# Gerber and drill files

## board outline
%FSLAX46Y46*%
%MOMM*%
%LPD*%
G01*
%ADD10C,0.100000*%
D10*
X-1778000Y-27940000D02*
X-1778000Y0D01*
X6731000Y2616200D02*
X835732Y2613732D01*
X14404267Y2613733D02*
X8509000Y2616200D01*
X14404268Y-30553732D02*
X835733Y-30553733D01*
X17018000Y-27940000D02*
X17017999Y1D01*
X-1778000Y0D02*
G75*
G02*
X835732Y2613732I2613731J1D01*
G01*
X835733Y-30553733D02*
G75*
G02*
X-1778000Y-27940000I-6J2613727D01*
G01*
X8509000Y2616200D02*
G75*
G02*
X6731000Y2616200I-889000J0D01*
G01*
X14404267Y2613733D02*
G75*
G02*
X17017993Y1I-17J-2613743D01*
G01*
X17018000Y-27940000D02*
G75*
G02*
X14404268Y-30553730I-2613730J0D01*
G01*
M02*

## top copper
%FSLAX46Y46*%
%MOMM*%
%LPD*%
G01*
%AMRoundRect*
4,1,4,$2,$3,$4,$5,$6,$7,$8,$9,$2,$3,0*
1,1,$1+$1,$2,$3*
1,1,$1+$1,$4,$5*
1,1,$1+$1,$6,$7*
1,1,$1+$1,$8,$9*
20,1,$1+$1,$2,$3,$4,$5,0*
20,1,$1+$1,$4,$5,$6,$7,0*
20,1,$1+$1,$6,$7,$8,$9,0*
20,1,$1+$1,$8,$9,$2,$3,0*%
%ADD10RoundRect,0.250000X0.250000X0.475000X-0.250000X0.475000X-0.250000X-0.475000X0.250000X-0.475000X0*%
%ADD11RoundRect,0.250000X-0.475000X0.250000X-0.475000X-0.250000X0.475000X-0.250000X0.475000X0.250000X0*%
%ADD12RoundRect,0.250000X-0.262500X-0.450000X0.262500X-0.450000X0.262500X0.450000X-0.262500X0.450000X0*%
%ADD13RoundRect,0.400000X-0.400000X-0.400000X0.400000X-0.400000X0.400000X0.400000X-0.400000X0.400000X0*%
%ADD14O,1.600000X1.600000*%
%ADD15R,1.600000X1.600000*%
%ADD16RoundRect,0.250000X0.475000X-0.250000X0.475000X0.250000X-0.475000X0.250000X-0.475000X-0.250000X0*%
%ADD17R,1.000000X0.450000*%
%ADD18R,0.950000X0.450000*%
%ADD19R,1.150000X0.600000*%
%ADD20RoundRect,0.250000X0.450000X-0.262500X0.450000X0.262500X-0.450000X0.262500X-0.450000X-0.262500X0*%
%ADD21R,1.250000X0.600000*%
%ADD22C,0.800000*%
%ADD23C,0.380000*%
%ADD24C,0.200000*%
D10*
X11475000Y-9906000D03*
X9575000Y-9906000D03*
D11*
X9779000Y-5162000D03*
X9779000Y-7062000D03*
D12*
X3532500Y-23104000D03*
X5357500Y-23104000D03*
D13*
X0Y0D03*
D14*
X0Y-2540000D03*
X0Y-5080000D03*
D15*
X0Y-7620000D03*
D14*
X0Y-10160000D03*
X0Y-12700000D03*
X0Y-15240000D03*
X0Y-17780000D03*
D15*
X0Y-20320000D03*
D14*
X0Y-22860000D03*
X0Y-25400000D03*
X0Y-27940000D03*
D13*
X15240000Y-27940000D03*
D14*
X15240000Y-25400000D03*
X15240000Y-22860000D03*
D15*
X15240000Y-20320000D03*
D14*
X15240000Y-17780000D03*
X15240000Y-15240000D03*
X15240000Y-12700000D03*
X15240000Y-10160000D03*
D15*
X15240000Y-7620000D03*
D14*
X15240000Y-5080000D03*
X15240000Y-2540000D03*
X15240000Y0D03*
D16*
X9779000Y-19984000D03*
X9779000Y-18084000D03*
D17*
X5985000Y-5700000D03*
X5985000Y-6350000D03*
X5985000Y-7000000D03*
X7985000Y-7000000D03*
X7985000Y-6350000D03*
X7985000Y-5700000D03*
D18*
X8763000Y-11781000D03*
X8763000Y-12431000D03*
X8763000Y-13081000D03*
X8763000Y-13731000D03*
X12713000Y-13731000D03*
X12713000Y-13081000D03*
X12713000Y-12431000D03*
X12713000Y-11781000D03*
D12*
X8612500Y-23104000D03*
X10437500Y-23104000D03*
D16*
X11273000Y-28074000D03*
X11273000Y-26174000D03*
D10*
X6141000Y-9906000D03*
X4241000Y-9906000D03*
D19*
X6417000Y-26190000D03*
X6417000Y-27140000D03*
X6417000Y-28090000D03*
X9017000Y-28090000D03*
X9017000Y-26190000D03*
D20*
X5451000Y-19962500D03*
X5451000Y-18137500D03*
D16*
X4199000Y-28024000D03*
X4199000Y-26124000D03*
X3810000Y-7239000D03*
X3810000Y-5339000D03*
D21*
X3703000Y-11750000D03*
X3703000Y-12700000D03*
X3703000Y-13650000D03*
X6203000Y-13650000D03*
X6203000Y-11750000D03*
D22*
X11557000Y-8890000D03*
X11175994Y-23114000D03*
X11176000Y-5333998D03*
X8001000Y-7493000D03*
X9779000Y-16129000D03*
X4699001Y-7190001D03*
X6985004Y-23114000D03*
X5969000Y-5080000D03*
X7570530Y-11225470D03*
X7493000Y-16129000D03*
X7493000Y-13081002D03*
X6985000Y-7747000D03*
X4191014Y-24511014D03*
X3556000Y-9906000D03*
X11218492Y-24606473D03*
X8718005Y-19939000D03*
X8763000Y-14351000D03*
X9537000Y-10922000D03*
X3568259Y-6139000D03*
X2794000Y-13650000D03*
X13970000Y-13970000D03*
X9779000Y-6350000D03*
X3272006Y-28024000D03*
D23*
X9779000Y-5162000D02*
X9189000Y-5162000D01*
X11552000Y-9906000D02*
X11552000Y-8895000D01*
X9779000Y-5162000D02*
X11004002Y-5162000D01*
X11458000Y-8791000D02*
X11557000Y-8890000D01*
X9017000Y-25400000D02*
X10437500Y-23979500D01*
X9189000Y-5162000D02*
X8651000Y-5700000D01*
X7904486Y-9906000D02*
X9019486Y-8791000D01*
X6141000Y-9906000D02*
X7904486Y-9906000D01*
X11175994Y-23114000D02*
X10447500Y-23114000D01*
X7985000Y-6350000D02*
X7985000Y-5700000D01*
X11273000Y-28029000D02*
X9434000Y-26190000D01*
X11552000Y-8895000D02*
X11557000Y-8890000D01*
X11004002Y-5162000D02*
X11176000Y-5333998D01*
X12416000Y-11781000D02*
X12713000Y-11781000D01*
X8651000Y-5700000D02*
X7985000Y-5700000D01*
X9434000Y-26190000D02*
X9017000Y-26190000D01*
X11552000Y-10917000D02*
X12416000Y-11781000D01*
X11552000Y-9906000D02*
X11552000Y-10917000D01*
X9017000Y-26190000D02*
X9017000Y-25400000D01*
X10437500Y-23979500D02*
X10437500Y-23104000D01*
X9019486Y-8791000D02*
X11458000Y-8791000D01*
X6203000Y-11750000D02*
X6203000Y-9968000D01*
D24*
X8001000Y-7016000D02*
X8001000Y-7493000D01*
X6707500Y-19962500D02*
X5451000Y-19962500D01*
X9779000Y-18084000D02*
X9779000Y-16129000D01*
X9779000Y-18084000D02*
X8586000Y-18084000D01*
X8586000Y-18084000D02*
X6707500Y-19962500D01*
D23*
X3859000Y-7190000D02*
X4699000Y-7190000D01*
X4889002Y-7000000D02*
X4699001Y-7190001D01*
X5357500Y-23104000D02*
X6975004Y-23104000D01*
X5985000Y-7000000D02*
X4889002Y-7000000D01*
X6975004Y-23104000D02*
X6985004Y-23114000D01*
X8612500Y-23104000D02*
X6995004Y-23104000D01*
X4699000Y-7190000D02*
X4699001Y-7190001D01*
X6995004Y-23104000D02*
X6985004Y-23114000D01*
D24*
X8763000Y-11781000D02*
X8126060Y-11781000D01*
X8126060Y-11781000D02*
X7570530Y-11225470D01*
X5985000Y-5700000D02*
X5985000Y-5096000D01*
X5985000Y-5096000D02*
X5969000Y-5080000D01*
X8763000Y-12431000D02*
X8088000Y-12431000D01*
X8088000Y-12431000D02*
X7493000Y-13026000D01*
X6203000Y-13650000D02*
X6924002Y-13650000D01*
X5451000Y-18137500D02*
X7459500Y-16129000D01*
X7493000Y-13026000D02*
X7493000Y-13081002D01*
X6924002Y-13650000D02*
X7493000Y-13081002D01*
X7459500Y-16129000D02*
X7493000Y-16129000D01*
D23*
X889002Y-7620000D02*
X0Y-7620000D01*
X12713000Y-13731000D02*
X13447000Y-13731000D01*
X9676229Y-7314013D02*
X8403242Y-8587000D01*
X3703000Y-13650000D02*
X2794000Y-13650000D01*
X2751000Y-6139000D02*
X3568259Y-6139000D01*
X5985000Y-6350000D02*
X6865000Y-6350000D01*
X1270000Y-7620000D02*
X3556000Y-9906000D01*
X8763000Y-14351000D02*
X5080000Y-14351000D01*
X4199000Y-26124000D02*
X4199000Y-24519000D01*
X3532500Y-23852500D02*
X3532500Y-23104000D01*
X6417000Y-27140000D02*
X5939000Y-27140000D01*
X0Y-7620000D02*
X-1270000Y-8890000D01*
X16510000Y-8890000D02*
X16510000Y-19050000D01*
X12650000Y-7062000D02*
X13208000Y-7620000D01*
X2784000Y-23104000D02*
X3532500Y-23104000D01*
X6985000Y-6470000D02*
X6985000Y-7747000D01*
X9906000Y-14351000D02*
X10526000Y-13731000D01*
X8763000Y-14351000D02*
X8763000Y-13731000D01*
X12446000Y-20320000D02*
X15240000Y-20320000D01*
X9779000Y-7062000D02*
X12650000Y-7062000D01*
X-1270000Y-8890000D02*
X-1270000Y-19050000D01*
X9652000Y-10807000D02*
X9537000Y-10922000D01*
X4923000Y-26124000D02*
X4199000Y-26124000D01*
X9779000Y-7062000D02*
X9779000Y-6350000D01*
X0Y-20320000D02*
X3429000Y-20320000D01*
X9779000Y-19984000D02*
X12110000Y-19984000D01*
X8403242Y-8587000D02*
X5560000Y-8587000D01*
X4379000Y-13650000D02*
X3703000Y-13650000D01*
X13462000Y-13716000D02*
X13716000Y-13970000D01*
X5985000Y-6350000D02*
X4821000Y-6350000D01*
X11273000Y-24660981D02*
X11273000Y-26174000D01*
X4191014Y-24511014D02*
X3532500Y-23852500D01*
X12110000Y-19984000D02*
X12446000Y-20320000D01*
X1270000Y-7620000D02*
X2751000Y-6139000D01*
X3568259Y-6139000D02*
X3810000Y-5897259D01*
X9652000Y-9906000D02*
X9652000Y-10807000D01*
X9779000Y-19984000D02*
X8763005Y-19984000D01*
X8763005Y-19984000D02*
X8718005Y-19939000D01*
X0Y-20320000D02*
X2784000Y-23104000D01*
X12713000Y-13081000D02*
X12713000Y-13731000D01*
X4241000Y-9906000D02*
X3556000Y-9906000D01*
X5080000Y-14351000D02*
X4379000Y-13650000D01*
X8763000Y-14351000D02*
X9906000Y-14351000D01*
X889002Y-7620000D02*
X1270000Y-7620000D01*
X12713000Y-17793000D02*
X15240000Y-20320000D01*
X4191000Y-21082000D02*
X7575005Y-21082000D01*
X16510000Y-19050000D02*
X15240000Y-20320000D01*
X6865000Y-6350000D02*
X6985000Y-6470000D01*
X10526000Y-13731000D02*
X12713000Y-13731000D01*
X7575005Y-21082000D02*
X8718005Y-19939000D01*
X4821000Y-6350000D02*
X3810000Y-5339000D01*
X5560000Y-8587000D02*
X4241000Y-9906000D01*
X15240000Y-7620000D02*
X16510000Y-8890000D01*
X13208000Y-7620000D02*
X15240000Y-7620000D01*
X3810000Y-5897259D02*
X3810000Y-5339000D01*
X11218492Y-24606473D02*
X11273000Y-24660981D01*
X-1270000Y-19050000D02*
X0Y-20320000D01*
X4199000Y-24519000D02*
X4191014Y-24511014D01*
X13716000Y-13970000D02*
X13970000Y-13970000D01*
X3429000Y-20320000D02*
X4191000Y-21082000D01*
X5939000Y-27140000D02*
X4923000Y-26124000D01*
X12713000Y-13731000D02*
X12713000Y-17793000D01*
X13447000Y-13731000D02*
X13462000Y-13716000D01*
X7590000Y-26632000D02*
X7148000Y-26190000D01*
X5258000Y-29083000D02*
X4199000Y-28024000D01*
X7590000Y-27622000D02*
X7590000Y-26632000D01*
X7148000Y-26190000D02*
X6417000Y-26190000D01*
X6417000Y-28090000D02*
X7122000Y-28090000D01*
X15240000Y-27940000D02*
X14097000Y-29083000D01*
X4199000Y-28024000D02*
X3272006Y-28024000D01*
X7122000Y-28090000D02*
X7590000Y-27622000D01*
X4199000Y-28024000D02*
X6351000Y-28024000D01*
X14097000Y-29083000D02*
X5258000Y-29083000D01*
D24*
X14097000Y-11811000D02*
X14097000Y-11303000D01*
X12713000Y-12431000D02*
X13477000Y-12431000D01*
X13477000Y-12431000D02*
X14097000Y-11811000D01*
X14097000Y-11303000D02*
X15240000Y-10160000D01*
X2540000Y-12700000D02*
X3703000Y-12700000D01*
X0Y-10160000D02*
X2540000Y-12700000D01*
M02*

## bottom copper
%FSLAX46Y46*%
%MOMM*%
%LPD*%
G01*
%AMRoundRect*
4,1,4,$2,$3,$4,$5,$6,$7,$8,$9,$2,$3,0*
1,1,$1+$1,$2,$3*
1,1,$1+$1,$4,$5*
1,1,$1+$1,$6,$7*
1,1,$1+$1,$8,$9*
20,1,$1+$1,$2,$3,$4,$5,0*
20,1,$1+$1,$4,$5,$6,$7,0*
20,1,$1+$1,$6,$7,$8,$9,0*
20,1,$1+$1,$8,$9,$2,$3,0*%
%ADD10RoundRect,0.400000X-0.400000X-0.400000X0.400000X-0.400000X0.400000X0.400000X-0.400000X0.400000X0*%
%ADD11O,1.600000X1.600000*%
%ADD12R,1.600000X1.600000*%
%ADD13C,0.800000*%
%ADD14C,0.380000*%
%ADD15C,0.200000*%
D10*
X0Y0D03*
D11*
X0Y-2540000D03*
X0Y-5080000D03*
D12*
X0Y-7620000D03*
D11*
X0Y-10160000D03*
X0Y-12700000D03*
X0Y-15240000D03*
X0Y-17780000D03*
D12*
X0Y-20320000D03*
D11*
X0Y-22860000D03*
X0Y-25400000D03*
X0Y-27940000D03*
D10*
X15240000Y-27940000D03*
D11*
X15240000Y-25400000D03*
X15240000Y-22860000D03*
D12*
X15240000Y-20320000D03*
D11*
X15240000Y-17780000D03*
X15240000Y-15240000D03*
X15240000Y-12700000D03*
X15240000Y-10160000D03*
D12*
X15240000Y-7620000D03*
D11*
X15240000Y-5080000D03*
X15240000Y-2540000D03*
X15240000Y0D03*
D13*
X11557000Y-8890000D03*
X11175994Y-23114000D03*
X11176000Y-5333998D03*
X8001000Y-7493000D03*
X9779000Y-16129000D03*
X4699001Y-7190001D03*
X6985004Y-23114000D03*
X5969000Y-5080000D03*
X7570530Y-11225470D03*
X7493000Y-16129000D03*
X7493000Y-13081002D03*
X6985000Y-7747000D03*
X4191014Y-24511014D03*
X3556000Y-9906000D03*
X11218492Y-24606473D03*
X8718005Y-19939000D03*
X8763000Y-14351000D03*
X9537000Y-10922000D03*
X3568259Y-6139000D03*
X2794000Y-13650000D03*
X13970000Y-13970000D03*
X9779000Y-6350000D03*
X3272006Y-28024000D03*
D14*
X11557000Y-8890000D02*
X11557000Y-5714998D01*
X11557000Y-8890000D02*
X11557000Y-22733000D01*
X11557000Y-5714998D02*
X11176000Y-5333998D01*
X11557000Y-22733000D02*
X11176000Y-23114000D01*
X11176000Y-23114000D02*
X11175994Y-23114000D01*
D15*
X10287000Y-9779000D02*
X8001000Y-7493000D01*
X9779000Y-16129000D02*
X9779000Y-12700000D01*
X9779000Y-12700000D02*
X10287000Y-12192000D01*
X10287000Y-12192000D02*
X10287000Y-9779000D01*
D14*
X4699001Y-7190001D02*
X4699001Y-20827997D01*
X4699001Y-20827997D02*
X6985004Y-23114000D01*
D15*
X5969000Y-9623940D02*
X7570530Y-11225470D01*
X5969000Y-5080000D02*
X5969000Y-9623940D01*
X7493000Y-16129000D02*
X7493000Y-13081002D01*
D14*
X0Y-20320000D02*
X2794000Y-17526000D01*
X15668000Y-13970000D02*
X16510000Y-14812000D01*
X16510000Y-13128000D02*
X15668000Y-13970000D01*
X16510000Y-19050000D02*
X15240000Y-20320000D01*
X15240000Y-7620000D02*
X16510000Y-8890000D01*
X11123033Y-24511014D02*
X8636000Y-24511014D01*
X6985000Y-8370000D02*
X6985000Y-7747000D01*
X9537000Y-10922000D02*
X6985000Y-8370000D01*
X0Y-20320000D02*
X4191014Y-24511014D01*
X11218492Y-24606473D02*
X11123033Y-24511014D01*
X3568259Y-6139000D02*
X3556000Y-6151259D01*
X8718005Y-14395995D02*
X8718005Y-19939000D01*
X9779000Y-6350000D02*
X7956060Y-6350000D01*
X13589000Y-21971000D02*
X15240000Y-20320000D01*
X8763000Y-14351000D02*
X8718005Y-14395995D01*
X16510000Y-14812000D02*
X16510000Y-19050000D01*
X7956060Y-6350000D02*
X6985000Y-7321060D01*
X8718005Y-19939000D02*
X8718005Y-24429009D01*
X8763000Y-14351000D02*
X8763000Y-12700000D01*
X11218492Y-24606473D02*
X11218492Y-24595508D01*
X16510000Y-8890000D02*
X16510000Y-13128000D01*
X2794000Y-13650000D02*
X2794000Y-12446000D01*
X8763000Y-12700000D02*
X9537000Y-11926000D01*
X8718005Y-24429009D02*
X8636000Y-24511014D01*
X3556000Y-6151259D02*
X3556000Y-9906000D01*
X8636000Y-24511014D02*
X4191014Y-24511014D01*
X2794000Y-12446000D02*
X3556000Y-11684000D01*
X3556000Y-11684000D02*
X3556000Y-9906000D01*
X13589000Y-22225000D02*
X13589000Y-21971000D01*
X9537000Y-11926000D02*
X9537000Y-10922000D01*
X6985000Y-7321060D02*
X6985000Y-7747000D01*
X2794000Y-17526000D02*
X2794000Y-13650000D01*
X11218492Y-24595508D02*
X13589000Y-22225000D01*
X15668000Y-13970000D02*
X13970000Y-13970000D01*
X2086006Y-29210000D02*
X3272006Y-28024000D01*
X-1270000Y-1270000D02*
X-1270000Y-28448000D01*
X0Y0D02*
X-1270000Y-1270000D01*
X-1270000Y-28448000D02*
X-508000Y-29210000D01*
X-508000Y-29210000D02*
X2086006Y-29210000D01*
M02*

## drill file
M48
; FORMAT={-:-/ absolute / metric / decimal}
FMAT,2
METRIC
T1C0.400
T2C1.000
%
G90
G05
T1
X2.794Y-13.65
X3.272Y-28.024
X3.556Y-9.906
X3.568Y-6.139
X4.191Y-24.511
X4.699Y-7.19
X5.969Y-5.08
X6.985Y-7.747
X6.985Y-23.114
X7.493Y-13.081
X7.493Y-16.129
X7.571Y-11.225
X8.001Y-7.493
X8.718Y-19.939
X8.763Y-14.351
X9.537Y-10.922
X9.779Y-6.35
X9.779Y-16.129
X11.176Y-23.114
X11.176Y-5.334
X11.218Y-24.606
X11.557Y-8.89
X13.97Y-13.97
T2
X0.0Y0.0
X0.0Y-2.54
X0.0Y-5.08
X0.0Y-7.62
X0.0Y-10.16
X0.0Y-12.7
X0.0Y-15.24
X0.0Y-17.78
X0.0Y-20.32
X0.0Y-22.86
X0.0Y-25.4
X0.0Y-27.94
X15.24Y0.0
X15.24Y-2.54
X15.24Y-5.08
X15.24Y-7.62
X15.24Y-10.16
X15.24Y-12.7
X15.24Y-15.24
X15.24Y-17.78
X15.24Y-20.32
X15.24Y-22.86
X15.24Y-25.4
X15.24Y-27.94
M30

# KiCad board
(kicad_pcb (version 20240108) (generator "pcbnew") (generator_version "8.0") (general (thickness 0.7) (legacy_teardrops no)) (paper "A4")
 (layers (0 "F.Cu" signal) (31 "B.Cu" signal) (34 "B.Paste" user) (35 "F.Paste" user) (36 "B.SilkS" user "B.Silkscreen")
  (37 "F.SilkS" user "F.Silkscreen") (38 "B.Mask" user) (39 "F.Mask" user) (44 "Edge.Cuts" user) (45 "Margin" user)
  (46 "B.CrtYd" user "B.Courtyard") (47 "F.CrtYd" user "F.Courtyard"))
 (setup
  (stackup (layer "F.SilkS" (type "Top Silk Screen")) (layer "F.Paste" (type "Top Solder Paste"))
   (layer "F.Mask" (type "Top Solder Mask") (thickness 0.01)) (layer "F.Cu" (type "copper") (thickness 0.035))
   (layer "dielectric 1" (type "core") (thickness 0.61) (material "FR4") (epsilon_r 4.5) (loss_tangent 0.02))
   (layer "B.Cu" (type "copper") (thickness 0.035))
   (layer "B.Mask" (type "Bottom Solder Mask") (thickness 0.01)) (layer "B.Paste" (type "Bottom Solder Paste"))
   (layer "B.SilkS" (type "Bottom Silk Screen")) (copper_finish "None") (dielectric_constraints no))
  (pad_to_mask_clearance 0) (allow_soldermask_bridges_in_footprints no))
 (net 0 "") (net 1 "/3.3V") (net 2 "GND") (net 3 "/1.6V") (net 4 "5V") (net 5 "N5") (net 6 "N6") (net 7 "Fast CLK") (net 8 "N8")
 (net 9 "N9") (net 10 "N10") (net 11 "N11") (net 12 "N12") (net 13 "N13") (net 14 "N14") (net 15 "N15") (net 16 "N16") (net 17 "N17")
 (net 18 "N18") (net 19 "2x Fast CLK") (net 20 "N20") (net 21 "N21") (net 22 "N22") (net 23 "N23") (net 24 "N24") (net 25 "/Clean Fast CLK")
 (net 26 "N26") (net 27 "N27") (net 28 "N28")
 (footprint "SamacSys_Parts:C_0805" (layer "F.Cu") (at 10.541 9.906 90)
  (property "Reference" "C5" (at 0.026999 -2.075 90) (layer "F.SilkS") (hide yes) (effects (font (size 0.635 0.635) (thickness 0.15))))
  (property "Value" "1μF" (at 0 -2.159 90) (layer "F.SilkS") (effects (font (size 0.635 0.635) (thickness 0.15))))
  (pad "1" smd roundrect (at 0 0.934 180) (size 1 1.45) (layers "F.Cu" "F.Paste" "F.Mask") (roundrect_rratio 0.25) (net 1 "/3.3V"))
  (pad "2" smd roundrect (at 0 -0.966 180) (size 1 1.45) (layers "F.Cu" "F.Paste" "F.Mask") (roundrect_rratio 0.25) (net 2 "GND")))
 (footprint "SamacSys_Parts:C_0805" (layer "F.Cu") (at 9.779 6.096 180)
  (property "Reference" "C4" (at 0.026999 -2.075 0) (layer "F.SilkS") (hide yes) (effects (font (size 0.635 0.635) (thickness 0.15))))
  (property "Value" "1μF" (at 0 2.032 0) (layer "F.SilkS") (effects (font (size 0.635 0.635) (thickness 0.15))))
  (pad "1" smd roundrect (at 0 0.934 270) (size 1 1.45) (layers "F.Cu" "F.Paste" "F.Mask") (roundrect_rratio 0.25) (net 1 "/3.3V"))
  (pad "2" smd roundrect (at 0 -0.966 270) (size 1 1.45) (layers "F.Cu" "F.Paste" "F.Mask") (roundrect_rratio 0.25) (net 2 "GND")))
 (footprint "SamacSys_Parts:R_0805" (layer "F.Cu") (at 4.445 23.114 -90)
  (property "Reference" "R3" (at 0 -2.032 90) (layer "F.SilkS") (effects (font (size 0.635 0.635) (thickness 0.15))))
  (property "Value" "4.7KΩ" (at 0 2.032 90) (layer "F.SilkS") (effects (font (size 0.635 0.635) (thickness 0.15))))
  (pad "1" smd roundrect (at -0.01 0.9125) (size 1.025 1.4) (layers "F.Cu" "F.Paste" "F.Mask") (roundrect_rratio 0.243902) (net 2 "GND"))
  (pad "2" smd roundrect (at -0.01 -0.9125) (size 1.025 1.4) (layers "F.Cu" "F.Paste" "F.Mask") (roundrect_rratio 0.243902) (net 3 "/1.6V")))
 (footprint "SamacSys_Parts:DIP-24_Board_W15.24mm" (layer "F.Cu") (at 0 0)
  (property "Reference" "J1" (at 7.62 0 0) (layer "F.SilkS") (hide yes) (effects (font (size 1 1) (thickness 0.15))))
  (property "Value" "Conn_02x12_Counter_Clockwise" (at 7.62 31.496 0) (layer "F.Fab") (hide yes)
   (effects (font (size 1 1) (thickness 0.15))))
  (fp_line (start -1.778 27.94) (end -1.778 0) (stroke (width 0.1) (type solid)) (layer "Edge.Cuts"))
  (fp_line (start 6.731 -2.6162) (end 0.835732 -2.613732) (stroke (width 0.1) (type solid)) (layer "Edge.Cuts"))
  (fp_line (start 14.404267 -2.613733) (end 8.509 -2.6162) (stroke (width 0.1) (type solid)) (layer "Edge.Cuts"))
  (fp_line (start 14.404268 30.553732) (end 0.835733 30.553733) (stroke (width 0.1) (type solid)) (layer "Edge.Cuts"))
  (fp_line (start 17.018 27.94) (end 17.017999 -0.000001) (stroke (width 0.1) (type solid)) (layer "Edge.Cuts"))
  (fp_arc (start -1.778 0) (mid -1.012456 -1.848188) (end 0.835732 -2.613732) (stroke (width 0.1) (type solid)) (layer "Edge.Cuts"))
  (fp_arc (start 0.835733 30.553733) (mid -1.012457 29.78819) (end -1.778 27.94) (stroke (width 0.1) (type solid)) (layer "Edge.Cuts"))
  (fp_arc (start 8.509 -2.6162) (mid 7.62 -1.7272) (end 6.731 -2.6162) (stroke (width 0.1) (type default)) (layer "Edge.Cuts"))
  (fp_arc (start 14.404267 -2.613733) (mid 16.252451 -1.848184) (end 17.017999 -0.000001) (stroke (width 0.1) (type solid))
   (layer "Edge.Cuts"))
  (fp_arc (start 17.018 27.94) (mid 16.252456 29.788187) (end 14.404268 30.553732) (stroke (width 0.1) (type solid)) (layer "Edge.Cuts"))
  (pad "1" thru_hole roundrect (at 0 0) (size 1.6 1.6) (drill 1) (layers "*.Cu" "*.Mask") (remove_unused_layers no) (roundrect_rratio 0.25)
   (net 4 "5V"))
  (pad "2" thru_hole oval (at 0 2.54) (size 1.6 1.6) (drill 1) (layers "*.Cu" "*.Mask") (remove_unused_layers no) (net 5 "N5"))
  (pad "3" thru_hole oval (at 0 5.08) (size 1.6 1.6) (drill 1) (layers "*.Cu" "*.Mask") (remove_unused_layers no) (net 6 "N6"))
  (pad "4" thru_hole rect (at 0 7.62) (size 1.6 1.6) (drill 1) (layers "*.Cu" "*.Mask") (remove_unused_layers no) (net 2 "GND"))
  (pad "5" thru_hole oval (at 0 10.16) (size 1.6 1.6) (drill 1) (layers "*.Cu" "*.Mask") (remove_unused_layers no) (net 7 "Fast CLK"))
  (pad "6" thru_hole oval (at 0 12.7) (size 1.6 1.6) (drill 1) (layers "*.Cu" "*.Mask") (remove_unused_layers no) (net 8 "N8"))
  (pad "7" thru_hole oval (at 0 15.24) (size 1.6 1.6) (drill 1) (layers "*.Cu" "*.Mask") (remove_unused_layers no) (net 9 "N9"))
  (pad "8" thru_hole oval (at 0 17.78) (size 1.6 1.6) (drill 1) (layers "*.Cu" "*.Mask") (remove_unused_layers no) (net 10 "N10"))
  (pad "9" thru_hole rect (at 0 20.32) (size 1.6 1.6) (drill 1) (layers "*.Cu" "*.Mask") (remove_unused_layers no) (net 2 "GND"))
  (pad "10" thru_hole oval (at 0 22.86) (size 1.6 1.6) (drill 1) (layers "*.Cu" "*.Mask") (remove_unused_layers no) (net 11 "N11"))
  (pad "11" thru_hole oval (at 0 25.4) (size 1.6 1.6) (drill 1) (layers "*.Cu" "*.Mask") (remove_unused_layers no) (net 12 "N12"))
  (pad "12" thru_hole oval (at 0 27.94) (size 1.6 1.6) (drill 1) (layers "*.Cu" "*.Mask") (remove_unused_layers no) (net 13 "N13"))
  (pad "13" thru_hole roundrect (at 15.24 27.94) (size 1.6 1.6) (drill 1) (layers "*.Cu" "*.Mask") (remove_unused_layers no)
   (roundrect_rratio 0.25) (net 4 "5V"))
  (pad "14" thru_hole oval (at 15.24 25.4) (size 1.6 1.6) (drill 1) (layers "*.Cu" "*.Mask") (remove_unused_layers no) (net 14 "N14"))
  (pad "15" thru_hole oval (at 15.24 22.86) (size 1.6 1.6) (drill 1) (layers "*.Cu" "*.Mask") (remove_unused_layers no) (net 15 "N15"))
  (pad "16" thru_hole rect (at 15.24 20.32) (size 1.6 1.6) (drill 1) (layers "*.Cu" "*.Mask") (remove_unused_layers no) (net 2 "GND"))
  (pad "17" thru_hole oval (at 15.24 17.78 180) (size 1.6 1.6) (drill 1) (layers "*.Cu" "*.Mask") (remove_unused_layers no) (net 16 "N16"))
  (pad "18" thru_hole oval (at 15.24 15.24 180) (size 1.6 1.6) (drill 1) (layers "*.Cu" "*.Mask") (remove_unused_layers no) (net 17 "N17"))
  (pad "19" thru_hole oval (at 15.24 12.7 180) (size 1.6 1.6) (drill 1) (layers "*.Cu" "*.Mask") (remove_unused_layers no) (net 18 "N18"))
  (pad "20" thru_hole oval (at 15.24 10.16 180) (size 1.6 1.6) (drill 1) (layers "*.Cu" "*.Mask") (remove_unused_layers no)
   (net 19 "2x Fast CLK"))
  (pad "21" thru_hole rect (at 15.24 7.62) (size 1.6 1.6) (drill 1) (layers "*.Cu" "*.Mask") (remove_unused_layers no) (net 2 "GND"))
  (pad "22" thru_hole oval (at 15.24 5.08) (size 1.6 1.6) (drill 1) (layers "*.Cu" "*.Mask") (remove_unused_layers no) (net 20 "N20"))
  (pad "23" thru_hole oval (at 15.24 2.54) (size 1.6 1.6) (drill 1) (layers "*.Cu" "*.Mask") (remove_unused_layers no) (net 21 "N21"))
  (pad "24" thru_hole oval (at 15.24 0) (size 1.6 1.6) (drill 1) (layers "*.Cu" "*.Mask") (remove_unused_layers no) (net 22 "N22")))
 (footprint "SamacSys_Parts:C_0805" (layer "F.Cu") (at 9.779 19.05)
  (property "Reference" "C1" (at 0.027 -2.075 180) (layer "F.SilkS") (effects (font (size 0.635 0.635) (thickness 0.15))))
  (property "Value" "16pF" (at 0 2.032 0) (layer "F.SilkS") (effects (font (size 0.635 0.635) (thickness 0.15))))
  (pad "1" smd roundrect (at 0 0.934 90) (size 1 1.45) (layers "F.Cu" "F.Paste" "F.Mask") (roundrect_rratio 0.25) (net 2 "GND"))
  (pad "2" smd roundrect (at 0 -0.966 90) (size 1 1.45) (layers "F.Cu" "F.Paste" "F.Mask") (roundrect_rratio 0.25) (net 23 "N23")))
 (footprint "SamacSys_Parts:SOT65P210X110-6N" (layer "F.Cu") (at 6.985 6.35)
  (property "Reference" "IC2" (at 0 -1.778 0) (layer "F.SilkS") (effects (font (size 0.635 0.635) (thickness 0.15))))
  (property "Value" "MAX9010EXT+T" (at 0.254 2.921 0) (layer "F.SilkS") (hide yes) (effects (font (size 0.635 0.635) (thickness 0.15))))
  (pad "1" smd rect (at -1 -0.65 90) (size 0.45 1) (layers "F.Cu" "F.Paste" "F.Mask") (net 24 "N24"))
  (pad "2" smd rect (at -1 0 90) (size 0.45 1) (layers "F.Cu" "F.Paste" "F.Mask") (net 2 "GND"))
  (pad "3" smd rect (at -1 0.65 90) (size 0.45 1) (layers "F.Cu" "F.Paste" "F.Mask") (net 3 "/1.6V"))
  (pad "4" smd rect (at 1 0.65 90) (size 0.45 1) (layers "F.Cu" "F.Paste" "F.Mask") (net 23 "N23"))
  (pad "5" smd rect (at 1 0 90) (size 0.45 1) (layers "F.Cu" "F.Paste" "F.Mask") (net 1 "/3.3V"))
  (pad "6" smd rect (at 1 -0.65 90) (size 0.45 1) (layers "F.Cu" "F.Paste" "F.Mask") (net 1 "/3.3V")))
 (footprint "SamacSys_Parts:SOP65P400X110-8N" (layer "F.Cu") (at 10.738 12.756)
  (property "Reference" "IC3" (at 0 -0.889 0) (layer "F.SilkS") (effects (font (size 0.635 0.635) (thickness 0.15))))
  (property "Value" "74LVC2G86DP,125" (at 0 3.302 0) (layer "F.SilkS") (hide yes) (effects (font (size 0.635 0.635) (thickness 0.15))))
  (pad "1" smd rect (at -1.975 -0.975 90) (size 0.45 0.95) (layers "F.Cu" "F.Paste" "F.Mask") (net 24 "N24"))
  (pad "2" smd rect (at -1.975 -0.325 90) (size 0.45 0.95) (layers "F.Cu" "F.Paste" "F.Mask") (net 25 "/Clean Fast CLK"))
  (pad "3" smd rect (at -1.975 0.325 90) (size 0.45 0.95) (layers "F.Cu" "F.Paste" "F.Mask") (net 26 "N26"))
  (pad "4" smd rect (at -1.975 0.975 90) (size 0.45 0.95) (layers "F.Cu" "F.Paste" "F.Mask") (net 2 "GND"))
  (pad "5" smd rect (at 1.975 0.975 90) (size 0.45 0.95) (layers "F.Cu" "F.Paste" "F.Mask") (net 2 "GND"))
  (pad "6" smd rect (at 1.975 0.325 90) (size 0.45 0.95) (layers "F.Cu" "F.Paste" "F.Mask") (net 2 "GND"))
  (pad "7" smd rect (at 1.975 -0.325 90) (size 0.45 0.95) (layers "F.Cu" "F.Paste" "F.Mask") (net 19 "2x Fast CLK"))
  (pad "8" smd rect (at 1.975 -0.975 90) (size 0.45 0.95) (layers "F.Cu" "F.Paste" "F.Mask") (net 1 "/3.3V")))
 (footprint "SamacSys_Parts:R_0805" (layer "F.Cu") (at 9.525 23.114 -90)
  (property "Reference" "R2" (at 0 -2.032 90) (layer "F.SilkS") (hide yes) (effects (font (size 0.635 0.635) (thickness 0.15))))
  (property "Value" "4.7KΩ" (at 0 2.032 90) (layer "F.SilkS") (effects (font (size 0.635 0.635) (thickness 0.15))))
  (pad "1" smd roundrect (at -0.01 0.9125) (size 1.025 1.4) (layers "F.Cu" "F.Paste" "F.Mask") (roundrect_rratio 0.243902) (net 3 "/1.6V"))
  (pad "2" smd roundrect (at -0.01 -0.9125) (size 1.025 1.4) (layers "F.Cu" "F.Paste" "F.Mask") (roundrect_rratio 0.243902) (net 1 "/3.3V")))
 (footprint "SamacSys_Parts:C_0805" (layer "F.Cu") (at 11.273 27.14)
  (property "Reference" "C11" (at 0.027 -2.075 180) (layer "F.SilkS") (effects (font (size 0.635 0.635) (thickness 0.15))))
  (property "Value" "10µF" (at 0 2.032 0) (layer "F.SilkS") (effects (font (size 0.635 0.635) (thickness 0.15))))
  (pad "1" smd roundrect (at 0 0.934 90) (size 1 1.45) (layers "F.Cu" "F.Paste" "F.Mask") (roundrect_rratio 0.25) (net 1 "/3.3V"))
  (pad "2" smd roundrect (at 0 -0.966 90) (size 1 1.45) (layers "F.Cu" "F.Paste" "F.Mask") (roundrect_rratio 0.25) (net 2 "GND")))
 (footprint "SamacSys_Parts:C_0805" (layer "F.Cu") (at 5.207 9.906 90)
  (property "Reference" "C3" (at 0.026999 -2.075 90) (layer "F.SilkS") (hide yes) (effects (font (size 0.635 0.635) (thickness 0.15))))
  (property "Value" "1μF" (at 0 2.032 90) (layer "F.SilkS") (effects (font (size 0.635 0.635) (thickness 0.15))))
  (pad "1" smd roundrect (at 0 0.934 180) (size 1 1.45) (layers "F.Cu" "F.Paste" "F.Mask") (roundrect_rratio 0.25) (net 1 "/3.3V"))
  (pad "2" smd roundrect (at 0 -0.966 180) (size 1 1.45) (layers "F.Cu" "F.Paste" "F.Mask") (roundrect_rratio 0.25) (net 2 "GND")))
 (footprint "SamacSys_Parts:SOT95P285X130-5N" (layer "F.Cu") (at 7.717 27.14)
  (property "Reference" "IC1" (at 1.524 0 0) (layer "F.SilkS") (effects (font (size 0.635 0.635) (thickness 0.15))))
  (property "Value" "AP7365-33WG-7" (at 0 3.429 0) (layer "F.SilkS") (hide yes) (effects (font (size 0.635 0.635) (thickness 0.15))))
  (pad "1" smd rect (at -1.3 -0.95 90) (size 0.6 1.15) (layers "F.Cu" "F.Paste" "F.Mask") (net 4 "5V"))
  (pad "2" smd rect (at -1.3 0 90) (size 0.6 1.15) (layers "F.Cu" "F.Paste" "F.Mask") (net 2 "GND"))
  (pad "3" smd rect (at -1.3 0.95 90) (size 0.6 1.15) (layers "F.Cu" "F.Paste" "F.Mask") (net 4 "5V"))
  (pad "4" smd rect (at 1.3 0.95 90) (size 0.6 1.15) (layers "F.Cu" "F.Paste" "F.Mask") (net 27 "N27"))
  (pad "5" smd rect (at 1.3 -0.95 90) (size 0.6 1.15) (layers "F.Cu" "F.Paste" "F.Mask") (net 1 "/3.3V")))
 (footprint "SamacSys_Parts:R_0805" (layer "F.Cu") (at 5.461 19.05)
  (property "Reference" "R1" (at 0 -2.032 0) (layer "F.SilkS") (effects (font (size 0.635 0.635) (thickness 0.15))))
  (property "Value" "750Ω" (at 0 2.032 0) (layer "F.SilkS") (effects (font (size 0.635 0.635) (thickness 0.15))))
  (pad "1" smd roundrect (at -0.01 0.9125 90) (size 1.025 1.4) (layers "F.Cu" "F.Paste" "F.Mask") (roundrect_rratio 0.243902) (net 23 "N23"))
  (pad "2" smd roundrect (at -0.01 -0.9125 90) (size 1.025 1.4) (layers "F.Cu" "F.Paste" "F.Mask") (roundrect_rratio 0.243902)
   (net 25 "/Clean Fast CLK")))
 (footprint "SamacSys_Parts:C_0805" (layer "F.Cu") (at 4.199 27.09)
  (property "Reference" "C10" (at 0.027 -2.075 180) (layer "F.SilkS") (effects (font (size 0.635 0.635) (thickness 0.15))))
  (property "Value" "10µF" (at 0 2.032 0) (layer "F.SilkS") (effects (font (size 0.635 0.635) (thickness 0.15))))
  (pad "1" smd roundrect (at 0 0.934 90) (size 1 1.45) (layers "F.Cu" "F.Paste" "F.Mask") (roundrect_rratio 0.25) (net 4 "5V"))
  (pad "2" smd roundrect (at 0 -0.966 90) (size 1 1.45) (layers "F.Cu" "F.Paste" "F.Mask") (roundrect_rratio 0.25) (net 2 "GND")))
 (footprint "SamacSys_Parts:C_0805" (layer "F.Cu") (at 3.81 6.305)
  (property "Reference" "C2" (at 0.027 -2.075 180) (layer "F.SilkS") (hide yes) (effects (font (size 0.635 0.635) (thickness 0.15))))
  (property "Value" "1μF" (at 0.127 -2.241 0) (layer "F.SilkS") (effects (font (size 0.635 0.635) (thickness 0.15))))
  (pad "1" smd roundrect (at 0 0.934 90) (size 1 1.45) (layers "F.Cu" "F.Paste" "F.Mask") (roundrect_rratio 0.25) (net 3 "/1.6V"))
  (pad "2" smd roundrect (at 0 -0.966 90) (size 1 1.45) (layers "F.Cu" "F.Paste" "F.Mask") (roundrect_rratio 0.25) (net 2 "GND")))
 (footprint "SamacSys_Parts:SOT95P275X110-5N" (layer "F.Cu") (at 4.953 12.7)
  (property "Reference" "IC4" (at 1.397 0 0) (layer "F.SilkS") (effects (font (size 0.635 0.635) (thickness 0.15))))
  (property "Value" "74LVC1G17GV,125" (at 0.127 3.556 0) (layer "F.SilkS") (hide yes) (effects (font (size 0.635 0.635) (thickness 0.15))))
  (pad "1" smd rect (at -1.25 -0.95 90) (size 0.6 1.25) (layers "F.Cu" "F.Paste" "F.Mask") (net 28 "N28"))
  (pad "2" smd rect (at -1.25 0 90) (size 0.6 1.25) (layers "F.Cu" "F.Paste" "F.Mask") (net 7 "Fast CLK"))
  (pad "3" smd rect (at -1.25 0.95 90) (size 0.6 1.25) (layers "F.Cu" "F.Paste" "F.Mask") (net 2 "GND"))
  (pad "4" smd rect (at 1.25 0.95 90) (size 0.6 1.25) (layers "F.Cu" "F.Paste" "F.Mask") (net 25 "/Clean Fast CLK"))
  (pad "5" smd rect (at 1.25 -0.95 90) (size 0.6 1.25) (layers "F.Cu" "F.Paste" "F.Mask") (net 1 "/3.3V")))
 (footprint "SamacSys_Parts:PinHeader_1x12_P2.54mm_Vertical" (layer "B.Cu") (at 0 0 180)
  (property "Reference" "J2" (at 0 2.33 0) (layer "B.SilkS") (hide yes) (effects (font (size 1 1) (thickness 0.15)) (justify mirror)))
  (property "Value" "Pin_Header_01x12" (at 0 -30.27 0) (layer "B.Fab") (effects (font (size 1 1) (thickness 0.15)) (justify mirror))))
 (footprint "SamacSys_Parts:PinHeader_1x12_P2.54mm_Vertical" (layer "B.Cu") (at 15.24 0 180)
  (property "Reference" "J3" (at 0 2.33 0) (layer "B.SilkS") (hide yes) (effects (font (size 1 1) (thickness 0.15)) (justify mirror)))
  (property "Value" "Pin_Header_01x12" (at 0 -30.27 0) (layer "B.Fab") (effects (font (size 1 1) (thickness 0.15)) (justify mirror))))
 (segment (start 9.779 5.162) (end 9.189 5.162) (width 0.38) (layer "F.Cu") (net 1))
 (segment (start 11.552 9.906) (end 11.552 8.895) (width 0.38) (layer "F.Cu") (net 1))
 (segment (start 9.779 5.162) (end 11.004002 5.162) (width 0.38) (layer "F.Cu") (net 1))
 (segment (start 11.458 8.791) (end 11.557 8.89) (width 0.38) (layer "F.Cu") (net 1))
 (segment (start 9.017 25.4) (end 10.4375 23.9795) (width 0.38) (layer "F.Cu") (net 1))
 (segment (start 9.189 5.162) (end 8.651 5.7) (width 0.38) (layer "F.Cu") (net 1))
 (segment (start 7.904486 9.906) (end 9.019486 8.791) (width 0.38) (layer "F.Cu") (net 1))
 (segment (start 6.141 9.906) (end 7.904486 9.906) (width 0.38) (layer "F.Cu") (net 1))
 (segment (start 11.175994 23.114) (end 10.4475 23.114) (width 0.38) (layer "F.Cu") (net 1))
 (segment (start 7.985 6.35) (end 7.985 5.7) (width 0.38) (layer "F.Cu") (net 1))
 (segment (start 11.273 28.029) (end 9.434 26.19) (width 0.38) (layer "F.Cu") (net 1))
 (segment (start 11.552 8.895) (end 11.557 8.89) (width 0.38) (layer "F.Cu") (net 1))
 (segment (start 11.004002 5.162) (end 11.176 5.333998) (width 0.38) (layer "F.Cu") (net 1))
 (segment (start 12.416 11.781) (end 12.713 11.781) (width 0.38) (layer "F.Cu") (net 1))
 (segment (start 8.651 5.7) (end 7.985 5.7) (width 0.38) (layer "F.Cu") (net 1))
 (segment (start 9.434 26.19) (end 9.017 26.19) (width 0.38) (layer "F.Cu") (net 1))
 (segment (start 11.552 10.917) (end 12.416 11.781) (width 0.38) (layer "F.Cu") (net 1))
 (segment (start 11.552 9.906) (end 11.552 10.917) (width 0.38) (layer "F.Cu") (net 1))
 (segment (start 9.017 26.19) (end 9.017 25.4) (width 0.38) (layer "F.Cu") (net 1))
 (segment (start 10.4375 23.9795) (end 10.4375 23.104) (width 0.38) (layer "F.Cu") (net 1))
 (segment (start 9.019486 8.791) (end 11.458 8.791) (width 0.38) (layer "F.Cu") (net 1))
 (segment (start 6.203 11.75) (end 6.203 9.968) (width 0.38) (layer "F.Cu") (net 1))
 (via (at 11.557 8.89) (size 0.8) (drill 0.4) (layers "F.Cu" "B.Cu") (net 1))
 (via (at 11.175994 23.114) (size 0.8) (drill 0.4) (layers "F.Cu" "B.Cu") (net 1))
 (via (at 11.176 5.333998) (size 0.8) (drill 0.4) (layers "F.Cu" "B.Cu") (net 1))
 (segment (start 11.557 8.89) (end 11.557 5.714998) (width 0.38) (layer "B.Cu") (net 1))
 (segment (start 11.557 8.89) (end 11.557 22.733) (width 0.38) (layer "B.Cu") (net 1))
 (segment (start 11.557 5.714998) (end 11.176 5.333998) (width 0.38) (layer "B.Cu") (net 1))
 (segment (start 11.557 22.733) (end 11.176 23.114) (width 0.38) (layer "B.Cu") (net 1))
 (segment (start 11.176 23.114) (end 11.175994 23.114) (width 0.38) (layer "B.Cu") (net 1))
 (segment (start 8.001 7.016) (end 8.001 7.493) (width 0.2) (layer "F.Cu") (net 23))
 (segment (start 6.7075 19.9625) (end 5.451 19.9625) (width 0.2) (layer "F.Cu") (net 23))
 (segment (start 9.779 18.084) (end 9.779 16.129) (width 0.2) (layer "F.Cu") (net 23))
 (segment (start 9.779 18.084) (end 8.586 18.084) (width 0.2) (layer "F.Cu") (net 23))
 (segment (start 8.586 18.084) (end 6.7075 19.9625) (width 0.2) (layer "F.Cu") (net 23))
 (via (at 8.001 7.493) (size 0.8) (drill 0.4) (layers "F.Cu" "B.Cu") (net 23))
 (via (at 9.779 16.129) (size 0.8) (drill 0.4) (layers "F.Cu" "B.Cu") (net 23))
 (segment (start 10.287 9.779) (end 8.001 7.493) (width 0.2) (layer "B.Cu") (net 23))
 (segment (start 9.779 16.129) (end 9.779 12.7) (width 0.2) (layer "B.Cu") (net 23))
 (segment (start 9.779 12.7) (end 10.287 12.192) (width 0.2) (layer "B.Cu") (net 23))
 (segment (start 10.287 12.192) (end 10.287 9.779) (width 0.2) (layer "B.Cu") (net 23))
 (segment (start 3.859 7.19) (end 4.699 7.19) (width 0.38) (layer "F.Cu") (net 3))
 (segment (start 4.889002 7) (end 4.699001 7.190001) (width 0.38) (layer "F.Cu") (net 3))
 (segment (start 5.3575 23.104) (end 6.975004 23.104) (width 0.38) (layer "F.Cu") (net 3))
 (segment (start 5.985 7) (end 4.889002 7) (width 0.38) (layer "F.Cu") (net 3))
 (segment (start 6.975004 23.104) (end 6.985004 23.114) (width 0.38) (layer "F.Cu") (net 3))
 (segment (start 8.6125 23.104) (end 6.995004 23.104) (width 0.38) (layer "F.Cu") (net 3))
 (segment (start 4.699 7.19) (end 4.699001 7.190001) (width 0.38) (layer "F.Cu") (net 3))
 (segment (start 6.995004 23.104) (end 6.985004 23.114) (width 0.38) (layer "F.Cu") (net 3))
 (via (at 4.699001 7.190001) (size 0.8) (drill 0.4) (layers "F.Cu" "B.Cu") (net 3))
 (via (at 6.985004 23.114) (size 0.8) (drill 0.4) (layers "F.Cu" "B.Cu") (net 3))
 (segment (start 4.699001 7.190001) (end 4.699001 20.827997) (width 0.38) (layer "B.Cu") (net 3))
 (segment (start 4.699001 20.827997) (end 6.985004 23.114) (width 0.38) (layer "B.Cu") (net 3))
 (segment (start 8.763 11.781) (end 8.12606 11.781) (width 0.2) (layer "F.Cu") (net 24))
 (segment (start 8.12606 11.781) (end 7.57053 11.22547) (width 0.2) (layer "F.Cu") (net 24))
 (segment (start 5.985 5.7) (end 5.985 5.096) (width 0.2) (layer "F.Cu") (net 24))
 (segment (start 5.985 5.096) (end 5.969 5.08) (width 0.2) (layer "F.Cu") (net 24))
 (via (at 5.969 5.08) (size 0.8) (drill 0.4) (layers "F.Cu" "B.Cu") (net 24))
 (via (at 7.57053 11.22547) (size 0.8) (drill 0.4) (layers "F.Cu" "B.Cu") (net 24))
 (segment (start 5.969 9.62394) (end 7.57053 11.22547) (width 0.2) (layer "B.Cu") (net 24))
 (segment (start 5.969 5.08) (end 5.969 9.62394) (width 0.2) (layer "B.Cu") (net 24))
 (segment (start 8.763 12.431) (end 8.088 12.431) (width 0.2) (layer "F.Cu") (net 25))
 (segment (start 8.088 12.431) (end 7.493 13.026) (width 0.2) (layer "F.Cu") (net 25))
 (segment (start 6.203 13.65) (end 6.924002 13.65) (width 0.2) (layer "F.Cu") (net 25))
 (segment (start 5.451 18.1375) (end 7.4595 16.129) (width 0.2) (layer "F.Cu") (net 25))
 (segment (start 7.493 13.026) (end 7.493 13.081002) (width 0.2) (layer "F.Cu") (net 25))
 (segment (start 6.924002 13.65) (end 7.493 13.081002) (width 0.2) (layer "F.Cu") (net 25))
 (segment (start 7.4595 16.129) (end 7.493 16.129) (width 0.2) (layer "F.Cu") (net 25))
 (via (at 7.493 16.129) (size 0.8) (drill 0.4) (layers "F.Cu" "B.Cu") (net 25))
 (via (at 7.493 13.081002) (size 0.8) (drill 0.4) (layers "F.Cu" "B.Cu") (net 25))
 (segment (start 7.493 16.129) (end 7.493 13.081002) (width 0.2) (layer "B.Cu") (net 25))
 (segment (start 0.889002 7.62) (end 0 7.62) (width 0.38) (layer "F.Cu") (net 2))
 (segment (start 12.713 13.731) (end 13.447 13.731) (width 0.38) (layer "F.Cu") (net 2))
 (segment (start 9.676229 7.314013) (end 8.403242 8.587) (width 0.38) (layer "F.Cu") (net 2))
 (segment (start 3.703 13.65) (end 2.794 13.65) (width 0.38) (layer "F.Cu") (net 2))
 (segment (start 2.751 6.139) (end 3.568259 6.139) (width 0.38) (layer "F.Cu") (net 2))
 (segment (start 5.985 6.35) (end 6.865 6.35) (width 0.38) (layer "F.Cu") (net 2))
 (segment (start 1.27 7.62) (end 3.556 9.906) (width 0.38) (layer "F.Cu") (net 2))
 (segment (start 8.763 14.351) (end 5.08 14.351) (width 0.38) (layer "F.Cu") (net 2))
 (segment (start 4.199 26.124) (end 4.199 24.519) (width 0.38) (layer "F.Cu") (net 2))
 (segment (start 3.5325 23.8525) (end 3.5325 23.104) (width 0.38) (layer "F.Cu") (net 2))
 (segment (start 6.417 27.14) (end 5.939 27.14) (width 0.38) (layer "F.Cu") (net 2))
 (segment (start 0 7.62) (end -1.27 8.89) (width 0.38) (layer "F.Cu") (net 2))
 (segment (start 16.51 8.89) (end 16.51 19.05) (width 0.38) (layer "F.Cu") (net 2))
 (segment (start 12.65 7.062) (end 13.208 7.62) (width 0.38) (layer "F.Cu") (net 2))
 (segment (start 2.784 23.104) (end 3.5325 23.104) (width 0.38) (layer "F.Cu") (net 2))
 (segment (start 6.985 6.47) (end 6.985 7.747) (width 0.38) (layer "F.Cu") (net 2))
 (segment (start 9.906 14.351) (end 10.526 13.731) (width 0.38) (layer "F.Cu") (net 2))
 (segment (start 8.763 14.351) (end 8.763 13.731) (width 0.38) (layer "F.Cu") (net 2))
 (segment (start 12.446 20.32) (end 15.24 20.32) (width 0.38) (layer "F.Cu") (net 2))
 (segment (start 9.779 7.062) (end 12.65 7.062) (width 0.38) (layer "F.Cu") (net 2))
 (segment (start -1.27 8.89) (end -1.27 19.05) (width 0.38) (layer "F.Cu") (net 2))
 (segment (start 9.652 10.807) (end 9.537 10.922) (width 0.38) (layer "F.Cu") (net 2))
 (segment (start 4.923 26.124) (end 4.199 26.124) (width 0.38) (layer "F.Cu") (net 2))
 (segment (start 9.779 7.062) (end 9.779 6.35) (width 0.38) (layer "F.Cu") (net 2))
 (segment (start 0 20.32) (end 3.429 20.32) (width 0.38) (layer "F.Cu") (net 2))
 (segment (start 9.779 19.984) (end 12.11 19.984) (width 0.38) (layer "F.Cu") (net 2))
 (segment (start 8.403242 8.587) (end 5.56 8.587) (width 0.38) (layer "F.Cu") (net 2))
 (segment (start 4.379 13.65) (end 3.703 13.65) (width 0.38) (layer "F.Cu") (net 2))
 (segment (start 13.462 13.716) (end 13.716 13.97) (width 0.38) (layer "F.Cu") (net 2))
 (segment (start 5.985 6.35) (end 4.821 6.35) (width 0.38) (layer "F.Cu") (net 2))
 (segment (start 11.273 24.660981) (end 11.273 26.174) (width 0.38) (layer "F.Cu") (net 2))
 (segment (start 4.191014 24.511014) (end 3.5325 23.8525) (width 0.38) (layer "F.Cu") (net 2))
 (segment (start 12.11 19.984) (end 12.446 20.32) (width 0.38) (layer "F.Cu") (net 2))
 (segment (start 1.27 7.62) (end 2.751 6.139) (width 0.38) (layer "F.Cu") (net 2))
 (segment (start 3.568259 6.139) (end 3.81 5.897259) (width 0.38) (layer "F.Cu") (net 2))
 (segment (start 9.652 9.906) (end 9.652 10.807) (width 0.38) (layer "F.Cu") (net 2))
 (segment (start 9.779 19.984) (end 8.763005 19.984) (width 0.38) (layer "F.Cu") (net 2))
 (segment (start 8.763005 19.984) (end 8.718005 19.939) (width 0.38) (layer "F.Cu") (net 2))
 (segment (start 0 20.32) (end 2.784 23.104) (width 0.38) (layer "F.Cu") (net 2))
 (segment (start 12.713 13.081) (end 12.713 13.731) (width 0.38) (layer "F.Cu") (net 2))
 (segment (start 4.241 9.906) (end 3.556 9.906) (width 0.38) (layer "F.Cu") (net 2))
 (segment (start 5.08 14.351) (end 4.379 13.65) (width 0.38) (layer "F.Cu") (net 2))
 (segment (start 8.763 14.351) (end 9.906 14.351) (width 0.38) (layer "F.Cu") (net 2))
 (segment (start 0.889002 7.62) (end 1.27 7.62) (width 0.38) (layer "F.Cu") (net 2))
 (segment (start 12.713 17.793) (end 15.24 20.32) (width 0.38) (layer "F.Cu") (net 2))
 (segment (start 4.191 21.082) (end 7.575005 21.082) (width 0.38) (layer "F.Cu") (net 2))
 (segment (start 16.51 19.05) (end 15.24 20.32) (width 0.38) (layer "F.Cu") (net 2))
 (segment (start 6.865 6.35) (end 6.985 6.47) (width 0.38) (layer "F.Cu") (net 2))
 (segment (start 10.526 13.731) (end 12.713 13.731) (width 0.38) (layer "F.Cu") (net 2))
 (segment (start 7.575005 21.082) (end 8.718005 19.939) (width 0.38) (layer "F.Cu") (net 2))
 (segment (start 4.821 6.35) (end 3.81 5.339) (width 0.38) (layer "F.Cu") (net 2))
 (segment (start 5.56 8.587) (end 4.241 9.906) (width 0.38) (layer "F.Cu") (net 2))
 (segment (start 15.24 7.62) (end 16.51 8.89) (width 0.38) (layer "F.Cu") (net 2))
 (segment (start 13.208 7.62) (end 15.24 7.62) (width 0.38) (layer "F.Cu") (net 2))
 (segment (start 3.81 5.897259) (end 3.81 5.339) (width 0.38) (layer "F.Cu") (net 2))
 (segment (start 11.218492 24.606473) (end 11.273 24.660981) (width 0.38) (layer "F.Cu") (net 2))
 (segment (start -1.27 19.05) (end 0 20.32) (width 0.38) (layer "F.Cu") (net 2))
 (segment (start 4.199 24.519) (end 4.191014 24.511014) (width 0.38) (layer "F.Cu") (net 2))
 (segment (start 13.716 13.97) (end 13.97 13.97) (width 0.38) (layer "F.Cu") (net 2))
 (segment (start 3.429 20.32) (end 4.191 21.082) (width 0.38) (layer "F.Cu") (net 2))
 (segment (start 5.939 27.14) (end 4.923 26.124) (width 0.38) (layer "F.Cu") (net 2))
 (segment (start 12.713 13.731) (end 12.713 17.793) (width 0.38) (layer "F.Cu") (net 2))
 (segment (start 13.447 13.731) (end 13.462 13.716) (width 0.38) (layer "F.Cu") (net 2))
 (via (at 6.985 7.747) (size 0.8) (drill 0.4) (layers "F.Cu" "B.Cu") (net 2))
 (via (at 4.191014 24.511014) (size 0.8) (drill 0.4) (layers "F.Cu" "B.Cu") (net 2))
 (via (at 3.556 9.906) (size 0.8) (drill 0.4) (layers "F.Cu" "B.Cu") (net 2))
 (via (at 11.218492 24.606473) (size 0.8) (drill 0.4) (layers "F.Cu" "B.Cu") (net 2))
 (via (at 8.718005 19.939) (size 0.8) (drill 0.4) (layers "F.Cu" "B.Cu") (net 2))
 (via (at 8.763 14.351) (size 0.8) (drill 0.4) (layers "F.Cu" "B.Cu") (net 2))
 (via (at 9.537 10.922) (size 0.8) (drill 0.4) (layers "F.Cu" "B.Cu") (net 2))
 (via (at 3.568259 6.139) (size 0.8) (drill 0.4) (layers "F.Cu" "B.Cu") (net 2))
 (via (at 2.794 13.65) (size 0.8) (drill 0.4) (layers "F.Cu" "B.Cu") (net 2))
 (via (at 13.97 13.97) (size 0.8) (drill 0.4) (layers "F.Cu" "B.Cu") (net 2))
 (via (at 9.779 6.35) (size 0.8) (drill 0.4) (layers "F.Cu" "B.Cu") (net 2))
 (segment (start 0 20.32) (end 2.794 17.526) (width 0.38) (layer "B.Cu") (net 2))
 (segment (start 15.668 13.97) (end 16.51 14.812) (width 0.38) (layer "B.Cu") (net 2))
 (segment (start 16.51 13.128) (end 15.668 13.97) (width 0.38) (layer "B.Cu") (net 2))
 (segment (start 16.51 19.05) (end 15.24 20.32) (width 0.38) (layer "B.Cu") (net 2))
 (segment (start 15.24 7.62) (end 16.51 8.89) (width 0.38) (layer "B.Cu") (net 2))
 (segment (start 11.123033 24.511014) (end 8.636 24.511014) (width 0.38) (layer "B.Cu") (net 2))
 (segment (start 6.985 8.37) (end 6.985 7.747) (width 0.38) (layer "B.Cu") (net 2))
 (segment (start 9.537 10.922) (end 6.985 8.37) (width 0.38) (layer "B.Cu") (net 2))
 (segment (start 0 20.32) (end 4.191014 24.511014) (width 0.38) (layer "B.Cu") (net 2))
 (segment (start 11.218492 24.606473) (end 11.123033 24.511014) (width 0.38) (layer "B.Cu") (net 2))
 (segment (start 3.568259 6.139) (end 3.556 6.151259) (width 0.38) (layer "B.Cu") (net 2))
 (segment (start 8.718005 14.395995) (end 8.718005 19.939) (width 0.38) (layer "B.Cu") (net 2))
 (segment (start 9.779 6.35) (end 7.95606 6.35) (width 0.38) (layer "B.Cu") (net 2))
 (segment (start 13.589 21.971) (end 15.24 20.32) (width 0.38) (layer "B.Cu") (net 2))
 (segment (start 8.763 14.351) (end 8.718005 14.395995) (width 0.38) (layer "B.Cu") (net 2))
 (segment (start 16.51 14.812) (end 16.51 19.05) (width 0.38) (layer "B.Cu") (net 2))
 (segment (start 7.95606 6.35) (end 6.985 7.32106) (width 0.38) (layer "B.Cu") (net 2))
 (segment (start 8.718005 19.939) (end 8.718005 24.429009) (width 0.38) (layer "B.Cu") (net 2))
 (segment (start 8.763 14.351) (end 8.763 12.7) (width 0.38) (layer "B.Cu") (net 2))
 (segment (start 11.218492 24.606473) (end 11.218492 24.595508) (width 0.38) (layer "B.Cu") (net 2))
 (segment (start 16.51 8.89) (end 16.51 13.128) (width 0.38) (layer "B.Cu") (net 2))
 (segment (start 2.794 13.65) (end 2.794 12.446) (width 0.38) (layer "B.Cu") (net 2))
 (segment (start 8.763 12.7) (end 9.537 11.926) (width 0.38) (layer "B.Cu") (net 2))
 (segment (start 8.718005 24.429009) (end 8.636 24.511014) (width 0.38) (layer "B.Cu") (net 2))
 (segment (start 3.556 6.151259) (end 3.556 9.906) (width 0.38) (layer "B.Cu") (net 2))
 (segment (start 8.636 24.511014) (end 4.191014 24.511014) (width 0.38) (layer "B.Cu") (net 2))
 (segment (start 2.794 12.446) (end 3.556 11.684) (width 0.38) (layer "B.Cu") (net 2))
 (segment (start 3.556 11.684) (end 3.556 9.906) (width 0.38) (layer "B.Cu") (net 2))
 (segment (start 13.589 22.225) (end 13.589 21.971) (width 0.38) (layer "B.Cu") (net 2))
 (segment (start 9.537 11.926) (end 9.537 10.922) (width 0.38) (layer "B.Cu") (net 2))
 (segment (start 6.985 7.32106) (end 6.985 7.747) (width 0.38) (layer "B.Cu") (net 2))
 (segment (start 2.794 17.526) (end 2.794 13.65) (width 0.38) (layer "B.Cu") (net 2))
 (segment (start 11.218492 24.595508) (end 13.589 22.225) (width 0.38) (layer "B.Cu") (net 2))
 (segment (start 15.668 13.97) (end 13.97 13.97) (width 0.38) (layer "B.Cu") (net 2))
 (segment (start 7.59 26.632) (end 7.148 26.19) (width 0.38) (layer "F.Cu") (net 4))
 (segment (start 5.258 29.083) (end 4.199 28.024) (width 0.38) (layer "F.Cu") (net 4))
 (segment (start 7.59 27.622) (end 7.59 26.632) (width 0.38) (layer "F.Cu") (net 4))
 (segment (start 7.148 26.19) (end 6.417 26.19) (width 0.38) (layer "F.Cu") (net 4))
 (segment (start 6.417 28.09) (end 7.122 28.09) (width 0.38) (layer "F.Cu") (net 4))
 (segment (start 15.24 27.94) (end 14.097 29.083) (width 0.38) (layer "F.Cu") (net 4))
 (segment (start 4.199 28.024) (end 3.272006 28.024) (width 0.38) (layer "F.Cu") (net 4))
 (segment (start 7.122 28.09) (end 7.59 27.622) (width 0.38) (layer "F.Cu") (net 4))
 (segment (start 4.199 28.024) (end 6.351 28.024) (width 0.38) (layer "F.Cu") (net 4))
 (segment (start 14.097 29.083) (end 5.258 29.083) (width 0.38) (layer "F.Cu") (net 4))
 (via (at 3.272006 28.024) (size 0.8) (drill 0.4) (layers "F.Cu" "B.Cu") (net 4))
 (segment (start 2.086006 29.21) (end 3.272006 28.024) (width 0.38) (layer "B.Cu") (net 4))
 (segment (start -1.27 1.27) (end -1.27 28.448) (width 0.38) (layer "B.Cu") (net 4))
 (segment (start 0 0) (end -1.27 1.27) (width 0.38) (layer "B.Cu") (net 4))
 (segment (start -1.27 28.448) (end -0.508 29.21) (width 0.38) (layer "B.Cu") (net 4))
 (segment (start -0.508 29.21) (end 2.086006 29.21) (width 0.38) (layer "B.Cu") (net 4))
 (segment (start 14.097 11.811) (end 14.097 11.303) (width 0.2) (layer "F.Cu") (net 19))
 (segment (start 12.713 12.431) (end 13.477 12.431) (width 0.2) (layer "F.Cu") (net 19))
 (segment (start 13.477 12.431) (end 14.097 11.811) (width 0.2) (layer "F.Cu") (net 19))
 (segment (start 14.097 11.303) (end 15.24 10.16) (width 0.2) (layer "F.Cu") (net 19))
 (segment (start 2.54 12.7) (end 3.703 12.7) (width 0.2) (layer "F.Cu") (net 7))
 (segment (start 0 10.16) (end 2.54 12.7) (width 0.2) (layer "F.Cu") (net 7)))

